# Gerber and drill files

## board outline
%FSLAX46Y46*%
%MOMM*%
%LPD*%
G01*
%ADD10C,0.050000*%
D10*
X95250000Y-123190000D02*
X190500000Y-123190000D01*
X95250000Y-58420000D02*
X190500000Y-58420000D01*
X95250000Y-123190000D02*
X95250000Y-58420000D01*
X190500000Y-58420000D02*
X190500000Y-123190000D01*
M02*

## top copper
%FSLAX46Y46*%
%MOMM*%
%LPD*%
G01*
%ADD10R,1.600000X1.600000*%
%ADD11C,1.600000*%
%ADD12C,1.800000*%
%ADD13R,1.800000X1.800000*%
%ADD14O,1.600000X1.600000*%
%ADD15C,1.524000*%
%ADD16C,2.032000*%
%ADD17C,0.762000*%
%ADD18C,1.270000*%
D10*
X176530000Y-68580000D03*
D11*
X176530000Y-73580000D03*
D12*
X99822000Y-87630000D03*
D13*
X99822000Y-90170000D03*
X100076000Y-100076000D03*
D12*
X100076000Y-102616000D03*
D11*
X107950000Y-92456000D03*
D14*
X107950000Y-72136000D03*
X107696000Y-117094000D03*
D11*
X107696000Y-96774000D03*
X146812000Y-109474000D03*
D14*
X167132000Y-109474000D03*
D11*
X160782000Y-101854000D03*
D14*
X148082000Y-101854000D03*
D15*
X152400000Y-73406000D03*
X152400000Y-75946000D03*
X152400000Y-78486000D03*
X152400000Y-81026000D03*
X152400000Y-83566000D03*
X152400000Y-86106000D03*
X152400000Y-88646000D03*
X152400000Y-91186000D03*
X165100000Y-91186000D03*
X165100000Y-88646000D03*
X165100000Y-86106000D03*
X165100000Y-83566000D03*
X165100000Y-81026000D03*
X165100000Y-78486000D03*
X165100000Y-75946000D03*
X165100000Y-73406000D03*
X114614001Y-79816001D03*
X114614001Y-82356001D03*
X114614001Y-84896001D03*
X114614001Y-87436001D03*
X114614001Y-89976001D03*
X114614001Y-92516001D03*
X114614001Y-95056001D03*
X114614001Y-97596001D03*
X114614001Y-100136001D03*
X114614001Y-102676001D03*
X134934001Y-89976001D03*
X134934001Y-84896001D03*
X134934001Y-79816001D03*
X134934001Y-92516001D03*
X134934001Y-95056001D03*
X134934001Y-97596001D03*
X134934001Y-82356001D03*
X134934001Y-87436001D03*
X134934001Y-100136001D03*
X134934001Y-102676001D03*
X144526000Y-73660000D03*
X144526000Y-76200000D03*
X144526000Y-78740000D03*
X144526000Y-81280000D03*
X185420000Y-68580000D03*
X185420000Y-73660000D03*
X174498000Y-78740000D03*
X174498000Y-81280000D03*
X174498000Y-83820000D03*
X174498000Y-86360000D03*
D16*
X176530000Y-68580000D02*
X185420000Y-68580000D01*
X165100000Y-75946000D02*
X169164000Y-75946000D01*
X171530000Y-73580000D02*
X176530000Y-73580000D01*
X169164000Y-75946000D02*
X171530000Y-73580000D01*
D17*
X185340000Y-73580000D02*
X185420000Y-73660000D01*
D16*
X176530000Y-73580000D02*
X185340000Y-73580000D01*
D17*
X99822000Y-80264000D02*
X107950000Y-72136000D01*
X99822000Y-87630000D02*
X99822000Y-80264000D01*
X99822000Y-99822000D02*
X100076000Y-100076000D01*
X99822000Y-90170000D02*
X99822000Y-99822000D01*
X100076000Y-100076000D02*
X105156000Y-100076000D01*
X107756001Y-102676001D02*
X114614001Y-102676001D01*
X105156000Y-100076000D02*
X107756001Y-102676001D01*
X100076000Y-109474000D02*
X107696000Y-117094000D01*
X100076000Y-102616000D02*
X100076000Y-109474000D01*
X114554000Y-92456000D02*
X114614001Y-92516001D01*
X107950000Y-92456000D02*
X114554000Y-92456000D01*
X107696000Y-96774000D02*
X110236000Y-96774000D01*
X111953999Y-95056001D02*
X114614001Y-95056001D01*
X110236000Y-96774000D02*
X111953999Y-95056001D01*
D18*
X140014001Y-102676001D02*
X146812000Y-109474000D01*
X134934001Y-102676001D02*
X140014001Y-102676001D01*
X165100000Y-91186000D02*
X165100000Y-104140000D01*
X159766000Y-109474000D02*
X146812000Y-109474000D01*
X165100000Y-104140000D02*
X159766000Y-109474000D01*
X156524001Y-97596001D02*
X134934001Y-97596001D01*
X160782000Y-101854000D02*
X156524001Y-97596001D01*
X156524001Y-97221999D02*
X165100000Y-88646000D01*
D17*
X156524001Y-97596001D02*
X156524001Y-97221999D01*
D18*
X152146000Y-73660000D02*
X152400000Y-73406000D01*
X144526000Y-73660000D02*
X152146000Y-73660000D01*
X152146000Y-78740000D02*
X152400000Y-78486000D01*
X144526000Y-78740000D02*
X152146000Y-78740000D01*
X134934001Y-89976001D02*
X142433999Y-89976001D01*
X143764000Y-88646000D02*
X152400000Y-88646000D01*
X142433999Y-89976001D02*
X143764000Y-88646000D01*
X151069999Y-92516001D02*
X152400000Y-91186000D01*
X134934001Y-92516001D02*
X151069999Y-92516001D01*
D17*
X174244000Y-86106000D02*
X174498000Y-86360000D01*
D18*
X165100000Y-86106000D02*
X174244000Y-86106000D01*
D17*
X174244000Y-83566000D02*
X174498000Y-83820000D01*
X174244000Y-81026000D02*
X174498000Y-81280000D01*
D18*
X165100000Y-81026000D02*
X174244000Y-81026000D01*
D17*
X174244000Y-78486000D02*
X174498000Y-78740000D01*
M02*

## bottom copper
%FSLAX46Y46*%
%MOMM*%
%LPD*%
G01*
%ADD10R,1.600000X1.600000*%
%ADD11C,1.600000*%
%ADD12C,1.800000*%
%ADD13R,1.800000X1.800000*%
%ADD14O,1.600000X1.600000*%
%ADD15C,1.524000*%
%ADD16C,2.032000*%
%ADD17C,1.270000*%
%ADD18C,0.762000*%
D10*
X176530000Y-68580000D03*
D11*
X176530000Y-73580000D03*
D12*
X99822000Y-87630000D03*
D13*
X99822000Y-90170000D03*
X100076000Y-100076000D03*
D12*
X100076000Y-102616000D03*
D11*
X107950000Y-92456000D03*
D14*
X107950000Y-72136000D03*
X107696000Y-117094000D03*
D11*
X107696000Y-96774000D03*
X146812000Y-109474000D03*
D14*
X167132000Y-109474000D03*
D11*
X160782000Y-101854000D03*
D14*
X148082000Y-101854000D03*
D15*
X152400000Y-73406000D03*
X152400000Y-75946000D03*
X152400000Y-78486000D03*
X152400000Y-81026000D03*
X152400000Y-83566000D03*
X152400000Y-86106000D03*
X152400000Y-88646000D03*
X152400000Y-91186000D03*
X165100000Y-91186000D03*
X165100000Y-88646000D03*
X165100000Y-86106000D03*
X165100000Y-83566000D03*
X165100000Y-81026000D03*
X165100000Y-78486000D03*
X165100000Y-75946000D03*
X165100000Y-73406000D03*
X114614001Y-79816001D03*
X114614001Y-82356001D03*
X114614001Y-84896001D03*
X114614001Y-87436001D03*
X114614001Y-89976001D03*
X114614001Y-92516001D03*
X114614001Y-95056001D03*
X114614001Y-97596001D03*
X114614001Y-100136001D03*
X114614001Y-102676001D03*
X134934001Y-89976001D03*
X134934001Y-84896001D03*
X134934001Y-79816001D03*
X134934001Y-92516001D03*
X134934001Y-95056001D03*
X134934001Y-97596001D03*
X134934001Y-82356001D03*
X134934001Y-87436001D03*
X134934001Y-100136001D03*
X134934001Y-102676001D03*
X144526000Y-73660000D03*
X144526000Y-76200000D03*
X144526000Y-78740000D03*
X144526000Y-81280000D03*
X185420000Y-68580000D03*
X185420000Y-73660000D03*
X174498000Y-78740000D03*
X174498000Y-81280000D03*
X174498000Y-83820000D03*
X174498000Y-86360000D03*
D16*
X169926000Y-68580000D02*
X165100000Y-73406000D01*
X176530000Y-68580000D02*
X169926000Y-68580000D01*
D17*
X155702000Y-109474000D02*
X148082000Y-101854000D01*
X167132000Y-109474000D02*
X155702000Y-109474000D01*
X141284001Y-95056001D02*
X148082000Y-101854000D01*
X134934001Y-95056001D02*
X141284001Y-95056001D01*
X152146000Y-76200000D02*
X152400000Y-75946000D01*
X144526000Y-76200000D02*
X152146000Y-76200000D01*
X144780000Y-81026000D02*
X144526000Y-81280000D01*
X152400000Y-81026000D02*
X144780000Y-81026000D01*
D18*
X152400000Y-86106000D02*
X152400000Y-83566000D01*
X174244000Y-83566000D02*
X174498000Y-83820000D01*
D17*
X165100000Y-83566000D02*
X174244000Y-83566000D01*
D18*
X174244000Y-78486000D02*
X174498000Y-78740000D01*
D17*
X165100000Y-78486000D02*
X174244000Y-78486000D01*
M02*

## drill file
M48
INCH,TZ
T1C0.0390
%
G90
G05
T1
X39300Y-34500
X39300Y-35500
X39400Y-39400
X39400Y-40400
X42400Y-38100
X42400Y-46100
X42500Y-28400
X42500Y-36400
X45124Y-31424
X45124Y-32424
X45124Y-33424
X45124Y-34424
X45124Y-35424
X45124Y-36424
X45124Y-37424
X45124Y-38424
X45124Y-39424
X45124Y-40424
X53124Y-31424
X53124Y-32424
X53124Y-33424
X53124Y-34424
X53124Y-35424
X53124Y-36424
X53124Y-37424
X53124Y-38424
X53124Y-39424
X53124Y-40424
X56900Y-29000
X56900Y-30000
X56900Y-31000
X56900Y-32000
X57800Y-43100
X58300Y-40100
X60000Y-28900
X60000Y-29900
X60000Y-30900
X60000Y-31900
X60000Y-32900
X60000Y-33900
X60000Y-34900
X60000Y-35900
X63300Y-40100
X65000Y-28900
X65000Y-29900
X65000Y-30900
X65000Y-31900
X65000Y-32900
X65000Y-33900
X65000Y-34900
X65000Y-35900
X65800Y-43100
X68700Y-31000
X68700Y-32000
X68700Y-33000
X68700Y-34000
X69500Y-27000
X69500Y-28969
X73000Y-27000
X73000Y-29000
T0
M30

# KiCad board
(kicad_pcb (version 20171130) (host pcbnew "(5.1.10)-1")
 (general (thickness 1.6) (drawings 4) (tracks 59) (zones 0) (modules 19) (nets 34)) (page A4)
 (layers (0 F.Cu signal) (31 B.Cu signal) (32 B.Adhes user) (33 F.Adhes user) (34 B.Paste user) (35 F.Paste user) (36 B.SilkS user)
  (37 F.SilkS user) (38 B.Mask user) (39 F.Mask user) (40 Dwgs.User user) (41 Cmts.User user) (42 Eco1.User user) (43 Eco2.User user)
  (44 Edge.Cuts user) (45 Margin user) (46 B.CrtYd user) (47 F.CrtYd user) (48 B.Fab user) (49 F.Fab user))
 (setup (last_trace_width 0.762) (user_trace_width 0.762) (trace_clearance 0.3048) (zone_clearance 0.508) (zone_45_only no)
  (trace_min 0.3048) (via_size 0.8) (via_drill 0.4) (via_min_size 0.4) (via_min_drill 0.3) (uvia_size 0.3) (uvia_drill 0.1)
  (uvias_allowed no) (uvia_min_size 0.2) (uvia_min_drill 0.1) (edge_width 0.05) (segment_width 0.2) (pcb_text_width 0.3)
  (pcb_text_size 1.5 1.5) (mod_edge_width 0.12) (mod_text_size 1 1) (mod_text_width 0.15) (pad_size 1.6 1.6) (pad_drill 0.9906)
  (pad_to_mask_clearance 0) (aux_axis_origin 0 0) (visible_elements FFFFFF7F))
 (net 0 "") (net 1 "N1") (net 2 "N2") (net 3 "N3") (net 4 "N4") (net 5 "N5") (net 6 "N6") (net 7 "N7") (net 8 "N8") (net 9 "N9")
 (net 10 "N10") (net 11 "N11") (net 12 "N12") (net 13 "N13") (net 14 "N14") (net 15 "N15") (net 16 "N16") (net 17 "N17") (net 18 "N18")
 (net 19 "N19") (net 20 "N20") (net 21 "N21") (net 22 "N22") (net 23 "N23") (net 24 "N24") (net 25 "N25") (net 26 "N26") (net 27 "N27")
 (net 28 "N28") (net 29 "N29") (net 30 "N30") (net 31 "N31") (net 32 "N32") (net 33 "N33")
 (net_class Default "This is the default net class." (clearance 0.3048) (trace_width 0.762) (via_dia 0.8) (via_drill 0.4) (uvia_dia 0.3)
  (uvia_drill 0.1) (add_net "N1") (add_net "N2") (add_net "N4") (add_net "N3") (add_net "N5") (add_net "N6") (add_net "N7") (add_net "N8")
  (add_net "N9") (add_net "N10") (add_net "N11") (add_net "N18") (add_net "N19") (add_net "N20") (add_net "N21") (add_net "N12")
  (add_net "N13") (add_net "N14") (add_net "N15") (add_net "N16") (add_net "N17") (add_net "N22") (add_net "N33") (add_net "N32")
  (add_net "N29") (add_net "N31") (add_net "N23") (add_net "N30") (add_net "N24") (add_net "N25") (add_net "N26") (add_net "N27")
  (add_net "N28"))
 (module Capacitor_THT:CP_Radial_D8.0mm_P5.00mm (layer F.Cu) (at 176.53 68.58 270)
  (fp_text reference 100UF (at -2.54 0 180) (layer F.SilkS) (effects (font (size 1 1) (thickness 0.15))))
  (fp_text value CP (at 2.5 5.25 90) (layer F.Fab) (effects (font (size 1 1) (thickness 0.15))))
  (pad 1 thru_hole rect (at 0 0 270) (size 1.6 1.6) (drill 0.9906) (layers *.Cu *.Mask) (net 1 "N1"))
  (pad 2 thru_hole circle (at 5 0 270) (size 1.6 1.6) (drill 0.9906) (layers *.Cu *.Mask) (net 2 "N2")))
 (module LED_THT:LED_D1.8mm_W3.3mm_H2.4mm (layer F.Cu) (at 99.822 90.17 90)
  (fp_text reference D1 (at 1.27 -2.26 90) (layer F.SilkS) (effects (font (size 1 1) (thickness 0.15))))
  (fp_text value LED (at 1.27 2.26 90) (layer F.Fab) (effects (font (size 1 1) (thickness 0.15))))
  (pad 2 thru_hole circle (at 2.54 0 90) (size 1.8 1.8) (drill 0.9906) (layers *.Cu *.Mask) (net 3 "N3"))
  (pad 1 thru_hole rect (at 0 0 90) (size 1.8 1.8) (drill 0.9906) (layers *.Cu *.Mask) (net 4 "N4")))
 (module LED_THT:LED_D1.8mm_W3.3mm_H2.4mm (layer F.Cu) (at 100.076 100.076 270)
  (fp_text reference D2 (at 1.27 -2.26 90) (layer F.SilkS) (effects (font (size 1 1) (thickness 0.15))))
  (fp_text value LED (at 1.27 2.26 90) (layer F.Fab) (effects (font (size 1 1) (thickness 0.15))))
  (pad 1 thru_hole rect (at 0 0 270) (size 1.8 1.8) (drill 0.9906) (layers *.Cu *.Mask) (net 4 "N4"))
  (pad 2 thru_hole circle (at 2.54 0 270) (size 1.8 1.8) (drill 0.9906) (layers *.Cu *.Mask) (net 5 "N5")))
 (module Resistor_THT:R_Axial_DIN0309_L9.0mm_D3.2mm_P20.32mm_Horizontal (layer F.Cu) (at 107.95 92.456 90)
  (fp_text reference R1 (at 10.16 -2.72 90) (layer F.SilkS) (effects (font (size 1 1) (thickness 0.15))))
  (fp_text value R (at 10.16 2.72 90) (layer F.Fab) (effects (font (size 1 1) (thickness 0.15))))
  (pad 1 thru_hole circle (at 0 0 90) (size 1.6 1.6) (drill 0.9906) (layers *.Cu *.Mask) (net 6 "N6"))
  (pad 2 thru_hole oval (at 20.32 0 90) (size 1.6 1.6) (drill 0.9906) (layers *.Cu *.Mask) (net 3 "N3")))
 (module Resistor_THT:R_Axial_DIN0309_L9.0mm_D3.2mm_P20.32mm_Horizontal (layer F.Cu) (at 107.696 96.774 270)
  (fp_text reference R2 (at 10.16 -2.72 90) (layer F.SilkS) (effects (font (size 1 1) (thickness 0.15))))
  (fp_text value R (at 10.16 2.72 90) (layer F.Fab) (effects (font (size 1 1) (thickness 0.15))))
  (pad 2 thru_hole oval (at 20.32 0 270) (size 1.6 1.6) (drill 0.9906) (layers *.Cu *.Mask) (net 5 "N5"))
  (pad 1 thru_hole circle (at 0 0 270) (size 1.6 1.6) (drill 0.9906) (layers *.Cu *.Mask) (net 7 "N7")))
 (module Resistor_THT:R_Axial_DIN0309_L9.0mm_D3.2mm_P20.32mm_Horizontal (layer F.Cu) (at 146.812 109.474)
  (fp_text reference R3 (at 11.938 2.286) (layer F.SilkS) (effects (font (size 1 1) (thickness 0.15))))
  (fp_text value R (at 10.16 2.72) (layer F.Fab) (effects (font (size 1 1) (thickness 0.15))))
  (pad 1 thru_hole circle (at 0 0) (size 1.6 1.6) (drill 0.9906) (layers *.Cu *.Mask) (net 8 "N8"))
  (pad 2 thru_hole oval (at 20.32 0) (size 1.6 1.6) (drill 0.9906) (layers *.Cu *.Mask) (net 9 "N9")))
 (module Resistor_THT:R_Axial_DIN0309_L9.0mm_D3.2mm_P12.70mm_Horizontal (layer F.Cu) (at 160.782 101.854 180)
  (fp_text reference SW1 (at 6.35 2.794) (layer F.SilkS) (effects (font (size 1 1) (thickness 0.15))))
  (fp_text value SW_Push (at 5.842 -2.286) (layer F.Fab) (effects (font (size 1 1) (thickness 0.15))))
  (pad 1 thru_hole circle (at 0 0 180) (size 1.6 1.6) (drill 0.9906) (layers *.Cu *.Mask) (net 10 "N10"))
  (pad 2 thru_hole oval (at 12.7 0 180) (size 1.6 1.6) (drill 0.9906) (layers *.Cu *.Mask) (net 9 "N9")))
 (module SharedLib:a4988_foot (layer F.Cu) (at 158.75 82.296)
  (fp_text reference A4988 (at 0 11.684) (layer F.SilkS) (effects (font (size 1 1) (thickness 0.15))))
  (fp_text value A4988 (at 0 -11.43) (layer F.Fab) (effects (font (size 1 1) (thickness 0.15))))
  (pad 1 thru_hole circle (at -6.35 -8.89) (size 1.524 1.524) (drill 0.9906) (layers *.Cu *.Mask) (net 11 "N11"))
  (pad 2 thru_hole circle (at -6.35 -6.35) (size 1.524 1.524) (drill 0.9906) (layers *.Cu *.Mask) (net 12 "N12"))
  (pad 3 thru_hole circle (at -6.35 -3.81) (size 1.524 1.524) (drill 0.9906) (layers *.Cu *.Mask) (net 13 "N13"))
  (pad 4 thru_hole circle (at -6.35 -1.27) (size 1.524 1.524) (drill 0.9906) (layers *.Cu *.Mask) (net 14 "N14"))
  (pad 5 thru_hole circle (at -6.35 1.27) (size 1.524 1.524) (drill 0.9906) (layers *.Cu *.Mask) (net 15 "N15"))
  (pad 6 thru_hole circle (at -6.35 3.81) (size 1.524 1.524) (drill 0.9906) (layers *.Cu *.Mask) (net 15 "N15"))
  (pad 7 thru_hole circle (at -6.35 6.35) (size 1.524 1.524) (drill 0.9906) (layers *.Cu *.Mask) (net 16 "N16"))
  (pad 8 thru_hole circle (at -6.35 8.89) (size 1.524 1.524) (drill 0.9906) (layers *.Cu *.Mask) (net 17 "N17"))
  (pad 9 thru_hole circle (at 6.35 8.89) (size 1.524 1.524) (drill 0.9906) (layers *.Cu *.Mask) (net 8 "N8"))
  (pad 10 thru_hole circle (at 6.35 6.35) (size 1.524 1.524) (drill 0.9906) (layers *.Cu *.Mask) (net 10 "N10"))
  (pad 11 thru_hole circle (at 6.35 3.81) (size 1.524 1.524) (drill 0.9906) (layers *.Cu *.Mask) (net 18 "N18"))
  (pad 12 thru_hole circle (at 6.35 1.27) (size 1.524 1.524) (drill 0.9906) (layers *.Cu *.Mask) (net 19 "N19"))
  (pad 13 thru_hole circle (at 6.35 -1.27) (size 1.524 1.524) (drill 0.9906) (layers *.Cu *.Mask) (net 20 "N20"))
  (pad 14 thru_hole circle (at 6.35 -3.81) (size 1.524 1.524) (drill 0.9906) (layers *.Cu *.Mask) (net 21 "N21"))
  (pad 15 thru_hole circle (at 6.35 -6.35) (size 1.524 1.524) (drill 0.9906) (layers *.Cu *.Mask) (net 2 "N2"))
  (pad 16 thru_hole circle (at 6.35 -8.89) (size 1.524 1.524) (drill 0.9906) (layers *.Cu *.Mask) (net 1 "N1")))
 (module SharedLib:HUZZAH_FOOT (layer F.Cu) (at 124.774001 91.246001)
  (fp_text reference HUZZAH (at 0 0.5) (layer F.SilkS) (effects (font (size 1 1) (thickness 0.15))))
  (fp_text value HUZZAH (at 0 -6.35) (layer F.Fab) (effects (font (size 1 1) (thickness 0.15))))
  (pad 1 thru_hole circle (at -10.16 -11.43) (size 1.524 1.524) (drill 0.9906) (layers *.Cu *.Mask) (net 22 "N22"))
  (pad 2 thru_hole circle (at -10.16 -8.89) (size 1.524 1.524) (drill 0.9906) (layers *.Cu *.Mask) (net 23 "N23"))
  (pad 3 thru_hole circle (at -10.16 -6.35) (size 1.524 1.524) (drill 0.9906) (layers *.Cu *.Mask) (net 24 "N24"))
  (pad 4 thru_hole circle (at -10.16 -3.81) (size 1.524 1.524) (drill 0.9906) (layers *.Cu *.Mask) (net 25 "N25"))
  (pad 5 thru_hole circle (at -10.16 -1.27) (size 1.524 1.524) (drill 0.9906) (layers *.Cu *.Mask) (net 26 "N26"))
  (pad 6 thru_hole circle (at -10.16 1.27) (size 1.524 1.524) (drill 0.9906) (layers *.Cu *.Mask) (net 6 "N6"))
  (pad 7 thru_hole circle (at -10.16 3.81) (size 1.524 1.524) (drill 0.9906) (layers *.Cu *.Mask) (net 7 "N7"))
  (pad 8 thru_hole circle (at -10.16 6.35) (size 1.524 1.524) (drill 0.9906) (layers *.Cu *.Mask) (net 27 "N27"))
  (pad 9 thru_hole circle (at -10.16 8.89) (size 1.524 1.524) (drill 0.9906) (layers *.Cu *.Mask) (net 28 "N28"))
  (pad 10 thru_hole circle (at -10.16 11.43) (size 1.524 1.524) (drill 0.9906) (layers *.Cu *.Mask) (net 4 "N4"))
  (pad 16 thru_hole circle (at 10.16 -1.27) (size 1.524 1.524) (drill 0.9906) (layers *.Cu *.Mask) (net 16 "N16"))
  (pad 18 thru_hole circle (at 10.16 -6.35) (size 1.524 1.524) (drill 0.9906) (layers *.Cu *.Mask) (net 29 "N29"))
  (pad 20 thru_hole circle (at 10.16 -11.43) (size 1.524 1.524) (drill 0.9906) (layers *.Cu *.Mask) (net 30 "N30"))
  (pad 15 thru_hole circle (at 10.16 1.27) (size 1.524 1.524) (drill 0.9906) (layers *.Cu *.Mask) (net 17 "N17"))
  (pad 14 thru_hole circle (at 10.16 3.81) (size 1.524 1.524) (drill 0.9906) (layers *.Cu *.Mask) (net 9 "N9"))
  (pad 13 thru_hole circle (at 10.16 6.35) (size 1.524 1.524) (drill 0.9906) (layers *.Cu *.Mask) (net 10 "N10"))
  (pad 19 thru_hole circle (at 10.16 -8.89) (size 1.524 1.524) (drill 0.9906) (layers *.Cu *.Mask) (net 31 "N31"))
  (pad 17 thru_hole circle (at 10.16 -3.81) (size 1.524 1.524) (drill 0.9906) (layers *.Cu *.Mask) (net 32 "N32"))
  (pad 12 thru_hole circle (at 10.16 8.89) (size 1.524 1.524) (drill 0.9906) (layers *.Cu *.Mask) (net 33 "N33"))
  (pad 11 thru_hole circle (at 10.16 11.43) (size 1.524 1.524) (drill 0.9906) (layers *.Cu *.Mask) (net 8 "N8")))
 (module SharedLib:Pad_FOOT (layer F.Cu) (at 144.526 73.66)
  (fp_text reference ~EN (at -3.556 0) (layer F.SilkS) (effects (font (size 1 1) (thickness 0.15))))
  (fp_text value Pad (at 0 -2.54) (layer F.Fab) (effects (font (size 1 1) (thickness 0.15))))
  (pad 1 thru_hole circle (at 0 0) (size 1.524 1.524) (drill 0.9906) (layers *.Cu *.Mask) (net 11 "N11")))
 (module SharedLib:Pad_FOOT (layer F.Cu) (at 144.526 76.2)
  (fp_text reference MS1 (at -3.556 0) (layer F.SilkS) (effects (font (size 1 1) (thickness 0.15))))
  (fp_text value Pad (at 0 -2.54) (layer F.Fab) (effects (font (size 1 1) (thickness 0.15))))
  (pad 1 thru_hole circle (at 0 0) (size 1.524 1.524) (drill 0.9906) (layers *.Cu *.Mask) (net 12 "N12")))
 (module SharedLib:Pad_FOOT (layer F.Cu) (at 144.526 78.74)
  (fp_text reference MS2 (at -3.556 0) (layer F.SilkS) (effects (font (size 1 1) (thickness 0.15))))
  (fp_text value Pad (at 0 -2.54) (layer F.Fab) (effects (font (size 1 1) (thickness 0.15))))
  (pad 1 thru_hole circle (at 0 0) (size 1.524 1.524) (drill 0.9906) (layers *.Cu *.Mask) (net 13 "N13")))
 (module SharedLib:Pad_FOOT (layer F.Cu) (at 144.526 81.28)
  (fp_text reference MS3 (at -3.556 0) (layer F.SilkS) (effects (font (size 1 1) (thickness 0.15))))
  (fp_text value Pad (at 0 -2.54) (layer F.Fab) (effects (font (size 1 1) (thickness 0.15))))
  (pad 1 thru_hole circle (at 0 0) (size 1.524 1.524) (drill 0.9906) (layers *.Cu *.Mask) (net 14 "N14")))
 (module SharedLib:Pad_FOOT (layer F.Cu) (at 185.42 68.58)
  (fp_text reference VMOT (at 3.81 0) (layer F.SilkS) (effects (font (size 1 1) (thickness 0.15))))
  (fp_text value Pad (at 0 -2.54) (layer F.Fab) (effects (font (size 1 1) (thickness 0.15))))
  (pad 1 thru_hole circle (at 0 0) (size 1.524 1.524) (drill 0.9906) (layers *.Cu *.Mask) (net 1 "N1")))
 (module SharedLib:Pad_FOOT (layer F.Cu) (at 185.42 73.66 180)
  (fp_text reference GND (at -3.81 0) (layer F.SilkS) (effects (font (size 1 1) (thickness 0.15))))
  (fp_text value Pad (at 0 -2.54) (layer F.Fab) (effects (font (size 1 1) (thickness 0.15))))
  (pad 1 thru_hole circle (at 0 0 180) (size 1.524 1.524) (drill 0.9906) (layers *.Cu *.Mask) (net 2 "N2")))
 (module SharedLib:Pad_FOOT (layer F.Cu) (at 174.498 78.74)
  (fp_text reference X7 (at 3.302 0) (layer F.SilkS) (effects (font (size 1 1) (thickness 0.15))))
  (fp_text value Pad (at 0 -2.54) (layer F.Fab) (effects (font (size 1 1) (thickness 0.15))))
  (pad 1 thru_hole circle (at 0 0) (size 1.524 1.524) (drill 0.9906) (layers *.Cu *.Mask) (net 21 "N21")))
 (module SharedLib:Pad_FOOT (layer F.Cu) (at 174.498 81.28)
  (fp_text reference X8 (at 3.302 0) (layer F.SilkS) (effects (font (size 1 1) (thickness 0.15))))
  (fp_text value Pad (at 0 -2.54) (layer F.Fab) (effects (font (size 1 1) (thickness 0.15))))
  (pad 1 thru_hole circle (at 0 0) (size 1.524 1.524) (drill 0.9906) (layers *.Cu *.Mask) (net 20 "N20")))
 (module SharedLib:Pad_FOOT (layer F.Cu) (at 174.498 83.82)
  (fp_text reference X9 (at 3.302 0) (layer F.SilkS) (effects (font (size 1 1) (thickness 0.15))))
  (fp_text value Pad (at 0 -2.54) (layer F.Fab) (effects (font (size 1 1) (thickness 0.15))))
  (pad 1 thru_hole circle (at 0 0) (size 1.524 1.524) (drill 0.9906) (layers *.Cu *.Mask) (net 19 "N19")))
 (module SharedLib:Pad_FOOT (layer F.Cu) (at 174.498 86.36)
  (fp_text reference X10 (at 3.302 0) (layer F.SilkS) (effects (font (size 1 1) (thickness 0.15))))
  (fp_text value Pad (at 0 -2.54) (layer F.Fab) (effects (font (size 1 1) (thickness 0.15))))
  (pad 1 thru_hole circle (at 0 0) (size 1.524 1.524) (drill 0.9906) (layers *.Cu *.Mask) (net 18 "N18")))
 (gr_line (start 95.25 123.19) (end 190.5 123.19) (layer Edge.Cuts) (width 0.05))
 (gr_line (start 95.25 58.42) (end 190.5 58.42) (layer Edge.Cuts) (width 0.05))
 (gr_line (start 95.25 123.19) (end 95.25 58.42) (layer Edge.Cuts) (width 0.05))
 (gr_line (start 190.5 58.42) (end 190.5 123.19) (layer Edge.Cuts) (width 0.05))
 (segment (start 176.53 68.58) (end 185.42 68.58) (width 2.032) (layer F.Cu) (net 1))
 (segment (start 169.926 68.58) (end 165.1 73.406) (width 2.032) (layer B.Cu) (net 1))
 (segment (start 176.53 68.58) (end 169.926 68.58) (width 2.032) (layer B.Cu) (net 1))
 (segment (start 165.1 75.946) (end 169.164 75.946) (width 2.032) (layer F.Cu) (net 2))
 (segment (start 171.53 73.58) (end 176.53 73.58) (width 2.032) (layer F.Cu) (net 2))
 (segment (start 169.164 75.946) (end 171.53 73.58) (width 2.032) (layer F.Cu) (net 2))
 (segment (start 185.34 73.58) (end 185.42 73.66) (width 0.762) (layer F.Cu) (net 2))
 (segment (start 176.53 73.58) (end 185.34 73.58) (width 2.032) (layer F.Cu) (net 2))
 (segment (start 99.822 80.264) (end 107.95 72.136) (width 0.762) (layer F.Cu) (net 3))
 (segment (start 99.822 87.63) (end 99.822 80.264) (width 0.762) (layer F.Cu) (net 3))
 (segment (start 99.822 99.822) (end 100.076 100.076) (width 0.762) (layer F.Cu) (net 4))
 (segment (start 99.822 90.17) (end 99.822 99.822) (width 0.762) (layer F.Cu) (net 4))
 (segment (start 100.076 100.076) (end 105.156 100.076) (width 0.762) (layer F.Cu) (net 4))
 (segment (start 107.756001 102.676001) (end 114.614001 102.676001) (width 0.762) (layer F.Cu) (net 4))
 (segment (start 105.156 100.076) (end 107.756001 102.676001) (width 0.762) (layer F.Cu) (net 4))
 (segment (start 100.076 109.474) (end 107.696 117.094) (width 0.762) (layer F.Cu) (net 5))
 (segment (start 100.076 102.616) (end 100.076 109.474) (width 0.762) (layer F.Cu) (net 5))
 (segment (start 114.554 92.456) (end 114.614001 92.516001) (width 0.762) (layer F.Cu) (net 6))
 (segment (start 107.95 92.456) (end 114.554 92.456) (width 0.762) (layer F.Cu) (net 6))
 (segment (start 107.696 96.774) (end 110.236 96.774) (width 0.762) (layer F.Cu) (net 7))
 (segment (start 111.953999 95.056001) (end 114.614001 95.056001) (width 0.762) (layer F.Cu) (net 7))
 (segment (start 110.236 96.774) (end 111.953999 95.056001) (width 0.762) (layer F.Cu) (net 7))
 (segment (start 140.014001 102.676001) (end 146.812 109.474) (width 1.27) (layer F.Cu) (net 8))
 (segment (start 134.934001 102.676001) (end 140.014001 102.676001) (width 1.27) (layer F.Cu) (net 8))
 (segment (start 165.1 91.186) (end 165.1 104.14) (width 1.27) (layer F.Cu) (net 8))
 (segment (start 159.766 109.474) (end 146.812 109.474) (width 1.27) (layer F.Cu) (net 8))
 (segment (start 165.1 104.14) (end 159.766 109.474) (width 1.27) (layer F.Cu) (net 8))
 (segment (start 155.702 109.474) (end 148.082 101.854) (width 1.27) (layer B.Cu) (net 9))
 (segment (start 167.132 109.474) (end 155.702 109.474) (width 1.27) (layer B.Cu) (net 9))
 (segment (start 141.284001 95.056001) (end 148.082 101.854) (width 1.27) (layer B.Cu) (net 9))
 (segment (start 134.934001 95.056001) (end 141.284001 95.056001) (width 1.27) (layer B.Cu) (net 9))
 (segment (start 156.524001 97.596001) (end 134.934001 97.596001) (width 1.27) (layer F.Cu) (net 10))
 (segment (start 160.782 101.854) (end 156.524001 97.596001) (width 1.27) (layer F.Cu) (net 10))
 (segment (start 156.524001 97.221999) (end 165.1 88.646) (width 1.27) (layer F.Cu) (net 10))
 (segment (start 156.524001 97.596001) (end 156.524001 97.221999) (width 0.762) (layer F.Cu) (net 10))
 (segment (start 152.146 73.66) (end 152.4 73.406) (width 1.27) (layer F.Cu) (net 11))
 (segment (start 144.526 73.66) (end 152.146 73.66) (width 1.27) (layer F.Cu) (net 11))
 (segment (start 152.146 76.2) (end 152.4 75.946) (width 1.27) (layer B.Cu) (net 12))
 (segment (start 144.526 76.2) (end 152.146 76.2) (width 1.27) (layer B.Cu) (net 12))
 (segment (start 152.146 78.74) (end 152.4 78.486) (width 1.27) (layer F.Cu) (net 13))
 (segment (start 144.526 78.74) (end 152.146 78.74) (width 1.27) (layer F.Cu) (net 13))
 (segment (start 144.78 81.026) (end 144.526 81.28) (width 1.27) (layer B.Cu) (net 14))
 (segment (start 152.4 81.026) (end 144.78 81.026) (width 1.27) (layer B.Cu) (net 14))
 (segment (start 152.4 86.106) (end 152.4 83.566) (width 0.762) (layer B.Cu) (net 15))
 (segment (start 134.934001 89.976001) (end 142.433999 89.976001) (width 1.27) (layer F.Cu) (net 16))
 (segment (start 143.764 88.646) (end 152.4 88.646) (width 1.27) (layer F.Cu) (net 16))
 (segment (start 142.433999 89.976001) (end 143.764 88.646) (width 1.27) (layer F.Cu) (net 16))
 (segment (start 151.069999 92.516001) (end 152.4 91.186) (width 1.27) (layer F.Cu) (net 17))
 (segment (start 134.934001 92.516001) (end 151.069999 92.516001) (width 1.27) (layer F.Cu) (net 17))
 (segment (start 174.244 86.106) (end 174.498 86.36) (width 0.762) (layer F.Cu) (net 18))
 (segment (start 165.1 86.106) (end 174.244 86.106) (width 1.27) (layer F.Cu) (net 18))
 (segment (start 174.244 83.566) (end 174.498 83.82) (width 0.762) (layer F.Cu) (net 19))
 (segment (start 174.244 83.566) (end 174.498 83.82) (width 0.762) (layer B.Cu) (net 19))
 (segment (start 165.1 83.566) (end 174.244 83.566) (width 1.27) (layer B.Cu) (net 19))
 (segment (start 174.244 81.026) (end 174.498 81.28) (width 0.762) (layer F.Cu) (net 20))
 (segment (start 165.1 81.026) (end 174.244 81.026) (width 1.27) (layer F.Cu) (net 20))
 (segment (start 174.244 78.486) (end 174.498 78.74) (width 0.762) (layer F.Cu) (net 21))
 (segment (start 174.244 78.486) (end 174.498 78.74) (width 0.762) (layer B.Cu) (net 21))
 (segment (start 165.1 78.486) (end 174.244 78.486) (width 1.27) (layer B.Cu) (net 21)))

